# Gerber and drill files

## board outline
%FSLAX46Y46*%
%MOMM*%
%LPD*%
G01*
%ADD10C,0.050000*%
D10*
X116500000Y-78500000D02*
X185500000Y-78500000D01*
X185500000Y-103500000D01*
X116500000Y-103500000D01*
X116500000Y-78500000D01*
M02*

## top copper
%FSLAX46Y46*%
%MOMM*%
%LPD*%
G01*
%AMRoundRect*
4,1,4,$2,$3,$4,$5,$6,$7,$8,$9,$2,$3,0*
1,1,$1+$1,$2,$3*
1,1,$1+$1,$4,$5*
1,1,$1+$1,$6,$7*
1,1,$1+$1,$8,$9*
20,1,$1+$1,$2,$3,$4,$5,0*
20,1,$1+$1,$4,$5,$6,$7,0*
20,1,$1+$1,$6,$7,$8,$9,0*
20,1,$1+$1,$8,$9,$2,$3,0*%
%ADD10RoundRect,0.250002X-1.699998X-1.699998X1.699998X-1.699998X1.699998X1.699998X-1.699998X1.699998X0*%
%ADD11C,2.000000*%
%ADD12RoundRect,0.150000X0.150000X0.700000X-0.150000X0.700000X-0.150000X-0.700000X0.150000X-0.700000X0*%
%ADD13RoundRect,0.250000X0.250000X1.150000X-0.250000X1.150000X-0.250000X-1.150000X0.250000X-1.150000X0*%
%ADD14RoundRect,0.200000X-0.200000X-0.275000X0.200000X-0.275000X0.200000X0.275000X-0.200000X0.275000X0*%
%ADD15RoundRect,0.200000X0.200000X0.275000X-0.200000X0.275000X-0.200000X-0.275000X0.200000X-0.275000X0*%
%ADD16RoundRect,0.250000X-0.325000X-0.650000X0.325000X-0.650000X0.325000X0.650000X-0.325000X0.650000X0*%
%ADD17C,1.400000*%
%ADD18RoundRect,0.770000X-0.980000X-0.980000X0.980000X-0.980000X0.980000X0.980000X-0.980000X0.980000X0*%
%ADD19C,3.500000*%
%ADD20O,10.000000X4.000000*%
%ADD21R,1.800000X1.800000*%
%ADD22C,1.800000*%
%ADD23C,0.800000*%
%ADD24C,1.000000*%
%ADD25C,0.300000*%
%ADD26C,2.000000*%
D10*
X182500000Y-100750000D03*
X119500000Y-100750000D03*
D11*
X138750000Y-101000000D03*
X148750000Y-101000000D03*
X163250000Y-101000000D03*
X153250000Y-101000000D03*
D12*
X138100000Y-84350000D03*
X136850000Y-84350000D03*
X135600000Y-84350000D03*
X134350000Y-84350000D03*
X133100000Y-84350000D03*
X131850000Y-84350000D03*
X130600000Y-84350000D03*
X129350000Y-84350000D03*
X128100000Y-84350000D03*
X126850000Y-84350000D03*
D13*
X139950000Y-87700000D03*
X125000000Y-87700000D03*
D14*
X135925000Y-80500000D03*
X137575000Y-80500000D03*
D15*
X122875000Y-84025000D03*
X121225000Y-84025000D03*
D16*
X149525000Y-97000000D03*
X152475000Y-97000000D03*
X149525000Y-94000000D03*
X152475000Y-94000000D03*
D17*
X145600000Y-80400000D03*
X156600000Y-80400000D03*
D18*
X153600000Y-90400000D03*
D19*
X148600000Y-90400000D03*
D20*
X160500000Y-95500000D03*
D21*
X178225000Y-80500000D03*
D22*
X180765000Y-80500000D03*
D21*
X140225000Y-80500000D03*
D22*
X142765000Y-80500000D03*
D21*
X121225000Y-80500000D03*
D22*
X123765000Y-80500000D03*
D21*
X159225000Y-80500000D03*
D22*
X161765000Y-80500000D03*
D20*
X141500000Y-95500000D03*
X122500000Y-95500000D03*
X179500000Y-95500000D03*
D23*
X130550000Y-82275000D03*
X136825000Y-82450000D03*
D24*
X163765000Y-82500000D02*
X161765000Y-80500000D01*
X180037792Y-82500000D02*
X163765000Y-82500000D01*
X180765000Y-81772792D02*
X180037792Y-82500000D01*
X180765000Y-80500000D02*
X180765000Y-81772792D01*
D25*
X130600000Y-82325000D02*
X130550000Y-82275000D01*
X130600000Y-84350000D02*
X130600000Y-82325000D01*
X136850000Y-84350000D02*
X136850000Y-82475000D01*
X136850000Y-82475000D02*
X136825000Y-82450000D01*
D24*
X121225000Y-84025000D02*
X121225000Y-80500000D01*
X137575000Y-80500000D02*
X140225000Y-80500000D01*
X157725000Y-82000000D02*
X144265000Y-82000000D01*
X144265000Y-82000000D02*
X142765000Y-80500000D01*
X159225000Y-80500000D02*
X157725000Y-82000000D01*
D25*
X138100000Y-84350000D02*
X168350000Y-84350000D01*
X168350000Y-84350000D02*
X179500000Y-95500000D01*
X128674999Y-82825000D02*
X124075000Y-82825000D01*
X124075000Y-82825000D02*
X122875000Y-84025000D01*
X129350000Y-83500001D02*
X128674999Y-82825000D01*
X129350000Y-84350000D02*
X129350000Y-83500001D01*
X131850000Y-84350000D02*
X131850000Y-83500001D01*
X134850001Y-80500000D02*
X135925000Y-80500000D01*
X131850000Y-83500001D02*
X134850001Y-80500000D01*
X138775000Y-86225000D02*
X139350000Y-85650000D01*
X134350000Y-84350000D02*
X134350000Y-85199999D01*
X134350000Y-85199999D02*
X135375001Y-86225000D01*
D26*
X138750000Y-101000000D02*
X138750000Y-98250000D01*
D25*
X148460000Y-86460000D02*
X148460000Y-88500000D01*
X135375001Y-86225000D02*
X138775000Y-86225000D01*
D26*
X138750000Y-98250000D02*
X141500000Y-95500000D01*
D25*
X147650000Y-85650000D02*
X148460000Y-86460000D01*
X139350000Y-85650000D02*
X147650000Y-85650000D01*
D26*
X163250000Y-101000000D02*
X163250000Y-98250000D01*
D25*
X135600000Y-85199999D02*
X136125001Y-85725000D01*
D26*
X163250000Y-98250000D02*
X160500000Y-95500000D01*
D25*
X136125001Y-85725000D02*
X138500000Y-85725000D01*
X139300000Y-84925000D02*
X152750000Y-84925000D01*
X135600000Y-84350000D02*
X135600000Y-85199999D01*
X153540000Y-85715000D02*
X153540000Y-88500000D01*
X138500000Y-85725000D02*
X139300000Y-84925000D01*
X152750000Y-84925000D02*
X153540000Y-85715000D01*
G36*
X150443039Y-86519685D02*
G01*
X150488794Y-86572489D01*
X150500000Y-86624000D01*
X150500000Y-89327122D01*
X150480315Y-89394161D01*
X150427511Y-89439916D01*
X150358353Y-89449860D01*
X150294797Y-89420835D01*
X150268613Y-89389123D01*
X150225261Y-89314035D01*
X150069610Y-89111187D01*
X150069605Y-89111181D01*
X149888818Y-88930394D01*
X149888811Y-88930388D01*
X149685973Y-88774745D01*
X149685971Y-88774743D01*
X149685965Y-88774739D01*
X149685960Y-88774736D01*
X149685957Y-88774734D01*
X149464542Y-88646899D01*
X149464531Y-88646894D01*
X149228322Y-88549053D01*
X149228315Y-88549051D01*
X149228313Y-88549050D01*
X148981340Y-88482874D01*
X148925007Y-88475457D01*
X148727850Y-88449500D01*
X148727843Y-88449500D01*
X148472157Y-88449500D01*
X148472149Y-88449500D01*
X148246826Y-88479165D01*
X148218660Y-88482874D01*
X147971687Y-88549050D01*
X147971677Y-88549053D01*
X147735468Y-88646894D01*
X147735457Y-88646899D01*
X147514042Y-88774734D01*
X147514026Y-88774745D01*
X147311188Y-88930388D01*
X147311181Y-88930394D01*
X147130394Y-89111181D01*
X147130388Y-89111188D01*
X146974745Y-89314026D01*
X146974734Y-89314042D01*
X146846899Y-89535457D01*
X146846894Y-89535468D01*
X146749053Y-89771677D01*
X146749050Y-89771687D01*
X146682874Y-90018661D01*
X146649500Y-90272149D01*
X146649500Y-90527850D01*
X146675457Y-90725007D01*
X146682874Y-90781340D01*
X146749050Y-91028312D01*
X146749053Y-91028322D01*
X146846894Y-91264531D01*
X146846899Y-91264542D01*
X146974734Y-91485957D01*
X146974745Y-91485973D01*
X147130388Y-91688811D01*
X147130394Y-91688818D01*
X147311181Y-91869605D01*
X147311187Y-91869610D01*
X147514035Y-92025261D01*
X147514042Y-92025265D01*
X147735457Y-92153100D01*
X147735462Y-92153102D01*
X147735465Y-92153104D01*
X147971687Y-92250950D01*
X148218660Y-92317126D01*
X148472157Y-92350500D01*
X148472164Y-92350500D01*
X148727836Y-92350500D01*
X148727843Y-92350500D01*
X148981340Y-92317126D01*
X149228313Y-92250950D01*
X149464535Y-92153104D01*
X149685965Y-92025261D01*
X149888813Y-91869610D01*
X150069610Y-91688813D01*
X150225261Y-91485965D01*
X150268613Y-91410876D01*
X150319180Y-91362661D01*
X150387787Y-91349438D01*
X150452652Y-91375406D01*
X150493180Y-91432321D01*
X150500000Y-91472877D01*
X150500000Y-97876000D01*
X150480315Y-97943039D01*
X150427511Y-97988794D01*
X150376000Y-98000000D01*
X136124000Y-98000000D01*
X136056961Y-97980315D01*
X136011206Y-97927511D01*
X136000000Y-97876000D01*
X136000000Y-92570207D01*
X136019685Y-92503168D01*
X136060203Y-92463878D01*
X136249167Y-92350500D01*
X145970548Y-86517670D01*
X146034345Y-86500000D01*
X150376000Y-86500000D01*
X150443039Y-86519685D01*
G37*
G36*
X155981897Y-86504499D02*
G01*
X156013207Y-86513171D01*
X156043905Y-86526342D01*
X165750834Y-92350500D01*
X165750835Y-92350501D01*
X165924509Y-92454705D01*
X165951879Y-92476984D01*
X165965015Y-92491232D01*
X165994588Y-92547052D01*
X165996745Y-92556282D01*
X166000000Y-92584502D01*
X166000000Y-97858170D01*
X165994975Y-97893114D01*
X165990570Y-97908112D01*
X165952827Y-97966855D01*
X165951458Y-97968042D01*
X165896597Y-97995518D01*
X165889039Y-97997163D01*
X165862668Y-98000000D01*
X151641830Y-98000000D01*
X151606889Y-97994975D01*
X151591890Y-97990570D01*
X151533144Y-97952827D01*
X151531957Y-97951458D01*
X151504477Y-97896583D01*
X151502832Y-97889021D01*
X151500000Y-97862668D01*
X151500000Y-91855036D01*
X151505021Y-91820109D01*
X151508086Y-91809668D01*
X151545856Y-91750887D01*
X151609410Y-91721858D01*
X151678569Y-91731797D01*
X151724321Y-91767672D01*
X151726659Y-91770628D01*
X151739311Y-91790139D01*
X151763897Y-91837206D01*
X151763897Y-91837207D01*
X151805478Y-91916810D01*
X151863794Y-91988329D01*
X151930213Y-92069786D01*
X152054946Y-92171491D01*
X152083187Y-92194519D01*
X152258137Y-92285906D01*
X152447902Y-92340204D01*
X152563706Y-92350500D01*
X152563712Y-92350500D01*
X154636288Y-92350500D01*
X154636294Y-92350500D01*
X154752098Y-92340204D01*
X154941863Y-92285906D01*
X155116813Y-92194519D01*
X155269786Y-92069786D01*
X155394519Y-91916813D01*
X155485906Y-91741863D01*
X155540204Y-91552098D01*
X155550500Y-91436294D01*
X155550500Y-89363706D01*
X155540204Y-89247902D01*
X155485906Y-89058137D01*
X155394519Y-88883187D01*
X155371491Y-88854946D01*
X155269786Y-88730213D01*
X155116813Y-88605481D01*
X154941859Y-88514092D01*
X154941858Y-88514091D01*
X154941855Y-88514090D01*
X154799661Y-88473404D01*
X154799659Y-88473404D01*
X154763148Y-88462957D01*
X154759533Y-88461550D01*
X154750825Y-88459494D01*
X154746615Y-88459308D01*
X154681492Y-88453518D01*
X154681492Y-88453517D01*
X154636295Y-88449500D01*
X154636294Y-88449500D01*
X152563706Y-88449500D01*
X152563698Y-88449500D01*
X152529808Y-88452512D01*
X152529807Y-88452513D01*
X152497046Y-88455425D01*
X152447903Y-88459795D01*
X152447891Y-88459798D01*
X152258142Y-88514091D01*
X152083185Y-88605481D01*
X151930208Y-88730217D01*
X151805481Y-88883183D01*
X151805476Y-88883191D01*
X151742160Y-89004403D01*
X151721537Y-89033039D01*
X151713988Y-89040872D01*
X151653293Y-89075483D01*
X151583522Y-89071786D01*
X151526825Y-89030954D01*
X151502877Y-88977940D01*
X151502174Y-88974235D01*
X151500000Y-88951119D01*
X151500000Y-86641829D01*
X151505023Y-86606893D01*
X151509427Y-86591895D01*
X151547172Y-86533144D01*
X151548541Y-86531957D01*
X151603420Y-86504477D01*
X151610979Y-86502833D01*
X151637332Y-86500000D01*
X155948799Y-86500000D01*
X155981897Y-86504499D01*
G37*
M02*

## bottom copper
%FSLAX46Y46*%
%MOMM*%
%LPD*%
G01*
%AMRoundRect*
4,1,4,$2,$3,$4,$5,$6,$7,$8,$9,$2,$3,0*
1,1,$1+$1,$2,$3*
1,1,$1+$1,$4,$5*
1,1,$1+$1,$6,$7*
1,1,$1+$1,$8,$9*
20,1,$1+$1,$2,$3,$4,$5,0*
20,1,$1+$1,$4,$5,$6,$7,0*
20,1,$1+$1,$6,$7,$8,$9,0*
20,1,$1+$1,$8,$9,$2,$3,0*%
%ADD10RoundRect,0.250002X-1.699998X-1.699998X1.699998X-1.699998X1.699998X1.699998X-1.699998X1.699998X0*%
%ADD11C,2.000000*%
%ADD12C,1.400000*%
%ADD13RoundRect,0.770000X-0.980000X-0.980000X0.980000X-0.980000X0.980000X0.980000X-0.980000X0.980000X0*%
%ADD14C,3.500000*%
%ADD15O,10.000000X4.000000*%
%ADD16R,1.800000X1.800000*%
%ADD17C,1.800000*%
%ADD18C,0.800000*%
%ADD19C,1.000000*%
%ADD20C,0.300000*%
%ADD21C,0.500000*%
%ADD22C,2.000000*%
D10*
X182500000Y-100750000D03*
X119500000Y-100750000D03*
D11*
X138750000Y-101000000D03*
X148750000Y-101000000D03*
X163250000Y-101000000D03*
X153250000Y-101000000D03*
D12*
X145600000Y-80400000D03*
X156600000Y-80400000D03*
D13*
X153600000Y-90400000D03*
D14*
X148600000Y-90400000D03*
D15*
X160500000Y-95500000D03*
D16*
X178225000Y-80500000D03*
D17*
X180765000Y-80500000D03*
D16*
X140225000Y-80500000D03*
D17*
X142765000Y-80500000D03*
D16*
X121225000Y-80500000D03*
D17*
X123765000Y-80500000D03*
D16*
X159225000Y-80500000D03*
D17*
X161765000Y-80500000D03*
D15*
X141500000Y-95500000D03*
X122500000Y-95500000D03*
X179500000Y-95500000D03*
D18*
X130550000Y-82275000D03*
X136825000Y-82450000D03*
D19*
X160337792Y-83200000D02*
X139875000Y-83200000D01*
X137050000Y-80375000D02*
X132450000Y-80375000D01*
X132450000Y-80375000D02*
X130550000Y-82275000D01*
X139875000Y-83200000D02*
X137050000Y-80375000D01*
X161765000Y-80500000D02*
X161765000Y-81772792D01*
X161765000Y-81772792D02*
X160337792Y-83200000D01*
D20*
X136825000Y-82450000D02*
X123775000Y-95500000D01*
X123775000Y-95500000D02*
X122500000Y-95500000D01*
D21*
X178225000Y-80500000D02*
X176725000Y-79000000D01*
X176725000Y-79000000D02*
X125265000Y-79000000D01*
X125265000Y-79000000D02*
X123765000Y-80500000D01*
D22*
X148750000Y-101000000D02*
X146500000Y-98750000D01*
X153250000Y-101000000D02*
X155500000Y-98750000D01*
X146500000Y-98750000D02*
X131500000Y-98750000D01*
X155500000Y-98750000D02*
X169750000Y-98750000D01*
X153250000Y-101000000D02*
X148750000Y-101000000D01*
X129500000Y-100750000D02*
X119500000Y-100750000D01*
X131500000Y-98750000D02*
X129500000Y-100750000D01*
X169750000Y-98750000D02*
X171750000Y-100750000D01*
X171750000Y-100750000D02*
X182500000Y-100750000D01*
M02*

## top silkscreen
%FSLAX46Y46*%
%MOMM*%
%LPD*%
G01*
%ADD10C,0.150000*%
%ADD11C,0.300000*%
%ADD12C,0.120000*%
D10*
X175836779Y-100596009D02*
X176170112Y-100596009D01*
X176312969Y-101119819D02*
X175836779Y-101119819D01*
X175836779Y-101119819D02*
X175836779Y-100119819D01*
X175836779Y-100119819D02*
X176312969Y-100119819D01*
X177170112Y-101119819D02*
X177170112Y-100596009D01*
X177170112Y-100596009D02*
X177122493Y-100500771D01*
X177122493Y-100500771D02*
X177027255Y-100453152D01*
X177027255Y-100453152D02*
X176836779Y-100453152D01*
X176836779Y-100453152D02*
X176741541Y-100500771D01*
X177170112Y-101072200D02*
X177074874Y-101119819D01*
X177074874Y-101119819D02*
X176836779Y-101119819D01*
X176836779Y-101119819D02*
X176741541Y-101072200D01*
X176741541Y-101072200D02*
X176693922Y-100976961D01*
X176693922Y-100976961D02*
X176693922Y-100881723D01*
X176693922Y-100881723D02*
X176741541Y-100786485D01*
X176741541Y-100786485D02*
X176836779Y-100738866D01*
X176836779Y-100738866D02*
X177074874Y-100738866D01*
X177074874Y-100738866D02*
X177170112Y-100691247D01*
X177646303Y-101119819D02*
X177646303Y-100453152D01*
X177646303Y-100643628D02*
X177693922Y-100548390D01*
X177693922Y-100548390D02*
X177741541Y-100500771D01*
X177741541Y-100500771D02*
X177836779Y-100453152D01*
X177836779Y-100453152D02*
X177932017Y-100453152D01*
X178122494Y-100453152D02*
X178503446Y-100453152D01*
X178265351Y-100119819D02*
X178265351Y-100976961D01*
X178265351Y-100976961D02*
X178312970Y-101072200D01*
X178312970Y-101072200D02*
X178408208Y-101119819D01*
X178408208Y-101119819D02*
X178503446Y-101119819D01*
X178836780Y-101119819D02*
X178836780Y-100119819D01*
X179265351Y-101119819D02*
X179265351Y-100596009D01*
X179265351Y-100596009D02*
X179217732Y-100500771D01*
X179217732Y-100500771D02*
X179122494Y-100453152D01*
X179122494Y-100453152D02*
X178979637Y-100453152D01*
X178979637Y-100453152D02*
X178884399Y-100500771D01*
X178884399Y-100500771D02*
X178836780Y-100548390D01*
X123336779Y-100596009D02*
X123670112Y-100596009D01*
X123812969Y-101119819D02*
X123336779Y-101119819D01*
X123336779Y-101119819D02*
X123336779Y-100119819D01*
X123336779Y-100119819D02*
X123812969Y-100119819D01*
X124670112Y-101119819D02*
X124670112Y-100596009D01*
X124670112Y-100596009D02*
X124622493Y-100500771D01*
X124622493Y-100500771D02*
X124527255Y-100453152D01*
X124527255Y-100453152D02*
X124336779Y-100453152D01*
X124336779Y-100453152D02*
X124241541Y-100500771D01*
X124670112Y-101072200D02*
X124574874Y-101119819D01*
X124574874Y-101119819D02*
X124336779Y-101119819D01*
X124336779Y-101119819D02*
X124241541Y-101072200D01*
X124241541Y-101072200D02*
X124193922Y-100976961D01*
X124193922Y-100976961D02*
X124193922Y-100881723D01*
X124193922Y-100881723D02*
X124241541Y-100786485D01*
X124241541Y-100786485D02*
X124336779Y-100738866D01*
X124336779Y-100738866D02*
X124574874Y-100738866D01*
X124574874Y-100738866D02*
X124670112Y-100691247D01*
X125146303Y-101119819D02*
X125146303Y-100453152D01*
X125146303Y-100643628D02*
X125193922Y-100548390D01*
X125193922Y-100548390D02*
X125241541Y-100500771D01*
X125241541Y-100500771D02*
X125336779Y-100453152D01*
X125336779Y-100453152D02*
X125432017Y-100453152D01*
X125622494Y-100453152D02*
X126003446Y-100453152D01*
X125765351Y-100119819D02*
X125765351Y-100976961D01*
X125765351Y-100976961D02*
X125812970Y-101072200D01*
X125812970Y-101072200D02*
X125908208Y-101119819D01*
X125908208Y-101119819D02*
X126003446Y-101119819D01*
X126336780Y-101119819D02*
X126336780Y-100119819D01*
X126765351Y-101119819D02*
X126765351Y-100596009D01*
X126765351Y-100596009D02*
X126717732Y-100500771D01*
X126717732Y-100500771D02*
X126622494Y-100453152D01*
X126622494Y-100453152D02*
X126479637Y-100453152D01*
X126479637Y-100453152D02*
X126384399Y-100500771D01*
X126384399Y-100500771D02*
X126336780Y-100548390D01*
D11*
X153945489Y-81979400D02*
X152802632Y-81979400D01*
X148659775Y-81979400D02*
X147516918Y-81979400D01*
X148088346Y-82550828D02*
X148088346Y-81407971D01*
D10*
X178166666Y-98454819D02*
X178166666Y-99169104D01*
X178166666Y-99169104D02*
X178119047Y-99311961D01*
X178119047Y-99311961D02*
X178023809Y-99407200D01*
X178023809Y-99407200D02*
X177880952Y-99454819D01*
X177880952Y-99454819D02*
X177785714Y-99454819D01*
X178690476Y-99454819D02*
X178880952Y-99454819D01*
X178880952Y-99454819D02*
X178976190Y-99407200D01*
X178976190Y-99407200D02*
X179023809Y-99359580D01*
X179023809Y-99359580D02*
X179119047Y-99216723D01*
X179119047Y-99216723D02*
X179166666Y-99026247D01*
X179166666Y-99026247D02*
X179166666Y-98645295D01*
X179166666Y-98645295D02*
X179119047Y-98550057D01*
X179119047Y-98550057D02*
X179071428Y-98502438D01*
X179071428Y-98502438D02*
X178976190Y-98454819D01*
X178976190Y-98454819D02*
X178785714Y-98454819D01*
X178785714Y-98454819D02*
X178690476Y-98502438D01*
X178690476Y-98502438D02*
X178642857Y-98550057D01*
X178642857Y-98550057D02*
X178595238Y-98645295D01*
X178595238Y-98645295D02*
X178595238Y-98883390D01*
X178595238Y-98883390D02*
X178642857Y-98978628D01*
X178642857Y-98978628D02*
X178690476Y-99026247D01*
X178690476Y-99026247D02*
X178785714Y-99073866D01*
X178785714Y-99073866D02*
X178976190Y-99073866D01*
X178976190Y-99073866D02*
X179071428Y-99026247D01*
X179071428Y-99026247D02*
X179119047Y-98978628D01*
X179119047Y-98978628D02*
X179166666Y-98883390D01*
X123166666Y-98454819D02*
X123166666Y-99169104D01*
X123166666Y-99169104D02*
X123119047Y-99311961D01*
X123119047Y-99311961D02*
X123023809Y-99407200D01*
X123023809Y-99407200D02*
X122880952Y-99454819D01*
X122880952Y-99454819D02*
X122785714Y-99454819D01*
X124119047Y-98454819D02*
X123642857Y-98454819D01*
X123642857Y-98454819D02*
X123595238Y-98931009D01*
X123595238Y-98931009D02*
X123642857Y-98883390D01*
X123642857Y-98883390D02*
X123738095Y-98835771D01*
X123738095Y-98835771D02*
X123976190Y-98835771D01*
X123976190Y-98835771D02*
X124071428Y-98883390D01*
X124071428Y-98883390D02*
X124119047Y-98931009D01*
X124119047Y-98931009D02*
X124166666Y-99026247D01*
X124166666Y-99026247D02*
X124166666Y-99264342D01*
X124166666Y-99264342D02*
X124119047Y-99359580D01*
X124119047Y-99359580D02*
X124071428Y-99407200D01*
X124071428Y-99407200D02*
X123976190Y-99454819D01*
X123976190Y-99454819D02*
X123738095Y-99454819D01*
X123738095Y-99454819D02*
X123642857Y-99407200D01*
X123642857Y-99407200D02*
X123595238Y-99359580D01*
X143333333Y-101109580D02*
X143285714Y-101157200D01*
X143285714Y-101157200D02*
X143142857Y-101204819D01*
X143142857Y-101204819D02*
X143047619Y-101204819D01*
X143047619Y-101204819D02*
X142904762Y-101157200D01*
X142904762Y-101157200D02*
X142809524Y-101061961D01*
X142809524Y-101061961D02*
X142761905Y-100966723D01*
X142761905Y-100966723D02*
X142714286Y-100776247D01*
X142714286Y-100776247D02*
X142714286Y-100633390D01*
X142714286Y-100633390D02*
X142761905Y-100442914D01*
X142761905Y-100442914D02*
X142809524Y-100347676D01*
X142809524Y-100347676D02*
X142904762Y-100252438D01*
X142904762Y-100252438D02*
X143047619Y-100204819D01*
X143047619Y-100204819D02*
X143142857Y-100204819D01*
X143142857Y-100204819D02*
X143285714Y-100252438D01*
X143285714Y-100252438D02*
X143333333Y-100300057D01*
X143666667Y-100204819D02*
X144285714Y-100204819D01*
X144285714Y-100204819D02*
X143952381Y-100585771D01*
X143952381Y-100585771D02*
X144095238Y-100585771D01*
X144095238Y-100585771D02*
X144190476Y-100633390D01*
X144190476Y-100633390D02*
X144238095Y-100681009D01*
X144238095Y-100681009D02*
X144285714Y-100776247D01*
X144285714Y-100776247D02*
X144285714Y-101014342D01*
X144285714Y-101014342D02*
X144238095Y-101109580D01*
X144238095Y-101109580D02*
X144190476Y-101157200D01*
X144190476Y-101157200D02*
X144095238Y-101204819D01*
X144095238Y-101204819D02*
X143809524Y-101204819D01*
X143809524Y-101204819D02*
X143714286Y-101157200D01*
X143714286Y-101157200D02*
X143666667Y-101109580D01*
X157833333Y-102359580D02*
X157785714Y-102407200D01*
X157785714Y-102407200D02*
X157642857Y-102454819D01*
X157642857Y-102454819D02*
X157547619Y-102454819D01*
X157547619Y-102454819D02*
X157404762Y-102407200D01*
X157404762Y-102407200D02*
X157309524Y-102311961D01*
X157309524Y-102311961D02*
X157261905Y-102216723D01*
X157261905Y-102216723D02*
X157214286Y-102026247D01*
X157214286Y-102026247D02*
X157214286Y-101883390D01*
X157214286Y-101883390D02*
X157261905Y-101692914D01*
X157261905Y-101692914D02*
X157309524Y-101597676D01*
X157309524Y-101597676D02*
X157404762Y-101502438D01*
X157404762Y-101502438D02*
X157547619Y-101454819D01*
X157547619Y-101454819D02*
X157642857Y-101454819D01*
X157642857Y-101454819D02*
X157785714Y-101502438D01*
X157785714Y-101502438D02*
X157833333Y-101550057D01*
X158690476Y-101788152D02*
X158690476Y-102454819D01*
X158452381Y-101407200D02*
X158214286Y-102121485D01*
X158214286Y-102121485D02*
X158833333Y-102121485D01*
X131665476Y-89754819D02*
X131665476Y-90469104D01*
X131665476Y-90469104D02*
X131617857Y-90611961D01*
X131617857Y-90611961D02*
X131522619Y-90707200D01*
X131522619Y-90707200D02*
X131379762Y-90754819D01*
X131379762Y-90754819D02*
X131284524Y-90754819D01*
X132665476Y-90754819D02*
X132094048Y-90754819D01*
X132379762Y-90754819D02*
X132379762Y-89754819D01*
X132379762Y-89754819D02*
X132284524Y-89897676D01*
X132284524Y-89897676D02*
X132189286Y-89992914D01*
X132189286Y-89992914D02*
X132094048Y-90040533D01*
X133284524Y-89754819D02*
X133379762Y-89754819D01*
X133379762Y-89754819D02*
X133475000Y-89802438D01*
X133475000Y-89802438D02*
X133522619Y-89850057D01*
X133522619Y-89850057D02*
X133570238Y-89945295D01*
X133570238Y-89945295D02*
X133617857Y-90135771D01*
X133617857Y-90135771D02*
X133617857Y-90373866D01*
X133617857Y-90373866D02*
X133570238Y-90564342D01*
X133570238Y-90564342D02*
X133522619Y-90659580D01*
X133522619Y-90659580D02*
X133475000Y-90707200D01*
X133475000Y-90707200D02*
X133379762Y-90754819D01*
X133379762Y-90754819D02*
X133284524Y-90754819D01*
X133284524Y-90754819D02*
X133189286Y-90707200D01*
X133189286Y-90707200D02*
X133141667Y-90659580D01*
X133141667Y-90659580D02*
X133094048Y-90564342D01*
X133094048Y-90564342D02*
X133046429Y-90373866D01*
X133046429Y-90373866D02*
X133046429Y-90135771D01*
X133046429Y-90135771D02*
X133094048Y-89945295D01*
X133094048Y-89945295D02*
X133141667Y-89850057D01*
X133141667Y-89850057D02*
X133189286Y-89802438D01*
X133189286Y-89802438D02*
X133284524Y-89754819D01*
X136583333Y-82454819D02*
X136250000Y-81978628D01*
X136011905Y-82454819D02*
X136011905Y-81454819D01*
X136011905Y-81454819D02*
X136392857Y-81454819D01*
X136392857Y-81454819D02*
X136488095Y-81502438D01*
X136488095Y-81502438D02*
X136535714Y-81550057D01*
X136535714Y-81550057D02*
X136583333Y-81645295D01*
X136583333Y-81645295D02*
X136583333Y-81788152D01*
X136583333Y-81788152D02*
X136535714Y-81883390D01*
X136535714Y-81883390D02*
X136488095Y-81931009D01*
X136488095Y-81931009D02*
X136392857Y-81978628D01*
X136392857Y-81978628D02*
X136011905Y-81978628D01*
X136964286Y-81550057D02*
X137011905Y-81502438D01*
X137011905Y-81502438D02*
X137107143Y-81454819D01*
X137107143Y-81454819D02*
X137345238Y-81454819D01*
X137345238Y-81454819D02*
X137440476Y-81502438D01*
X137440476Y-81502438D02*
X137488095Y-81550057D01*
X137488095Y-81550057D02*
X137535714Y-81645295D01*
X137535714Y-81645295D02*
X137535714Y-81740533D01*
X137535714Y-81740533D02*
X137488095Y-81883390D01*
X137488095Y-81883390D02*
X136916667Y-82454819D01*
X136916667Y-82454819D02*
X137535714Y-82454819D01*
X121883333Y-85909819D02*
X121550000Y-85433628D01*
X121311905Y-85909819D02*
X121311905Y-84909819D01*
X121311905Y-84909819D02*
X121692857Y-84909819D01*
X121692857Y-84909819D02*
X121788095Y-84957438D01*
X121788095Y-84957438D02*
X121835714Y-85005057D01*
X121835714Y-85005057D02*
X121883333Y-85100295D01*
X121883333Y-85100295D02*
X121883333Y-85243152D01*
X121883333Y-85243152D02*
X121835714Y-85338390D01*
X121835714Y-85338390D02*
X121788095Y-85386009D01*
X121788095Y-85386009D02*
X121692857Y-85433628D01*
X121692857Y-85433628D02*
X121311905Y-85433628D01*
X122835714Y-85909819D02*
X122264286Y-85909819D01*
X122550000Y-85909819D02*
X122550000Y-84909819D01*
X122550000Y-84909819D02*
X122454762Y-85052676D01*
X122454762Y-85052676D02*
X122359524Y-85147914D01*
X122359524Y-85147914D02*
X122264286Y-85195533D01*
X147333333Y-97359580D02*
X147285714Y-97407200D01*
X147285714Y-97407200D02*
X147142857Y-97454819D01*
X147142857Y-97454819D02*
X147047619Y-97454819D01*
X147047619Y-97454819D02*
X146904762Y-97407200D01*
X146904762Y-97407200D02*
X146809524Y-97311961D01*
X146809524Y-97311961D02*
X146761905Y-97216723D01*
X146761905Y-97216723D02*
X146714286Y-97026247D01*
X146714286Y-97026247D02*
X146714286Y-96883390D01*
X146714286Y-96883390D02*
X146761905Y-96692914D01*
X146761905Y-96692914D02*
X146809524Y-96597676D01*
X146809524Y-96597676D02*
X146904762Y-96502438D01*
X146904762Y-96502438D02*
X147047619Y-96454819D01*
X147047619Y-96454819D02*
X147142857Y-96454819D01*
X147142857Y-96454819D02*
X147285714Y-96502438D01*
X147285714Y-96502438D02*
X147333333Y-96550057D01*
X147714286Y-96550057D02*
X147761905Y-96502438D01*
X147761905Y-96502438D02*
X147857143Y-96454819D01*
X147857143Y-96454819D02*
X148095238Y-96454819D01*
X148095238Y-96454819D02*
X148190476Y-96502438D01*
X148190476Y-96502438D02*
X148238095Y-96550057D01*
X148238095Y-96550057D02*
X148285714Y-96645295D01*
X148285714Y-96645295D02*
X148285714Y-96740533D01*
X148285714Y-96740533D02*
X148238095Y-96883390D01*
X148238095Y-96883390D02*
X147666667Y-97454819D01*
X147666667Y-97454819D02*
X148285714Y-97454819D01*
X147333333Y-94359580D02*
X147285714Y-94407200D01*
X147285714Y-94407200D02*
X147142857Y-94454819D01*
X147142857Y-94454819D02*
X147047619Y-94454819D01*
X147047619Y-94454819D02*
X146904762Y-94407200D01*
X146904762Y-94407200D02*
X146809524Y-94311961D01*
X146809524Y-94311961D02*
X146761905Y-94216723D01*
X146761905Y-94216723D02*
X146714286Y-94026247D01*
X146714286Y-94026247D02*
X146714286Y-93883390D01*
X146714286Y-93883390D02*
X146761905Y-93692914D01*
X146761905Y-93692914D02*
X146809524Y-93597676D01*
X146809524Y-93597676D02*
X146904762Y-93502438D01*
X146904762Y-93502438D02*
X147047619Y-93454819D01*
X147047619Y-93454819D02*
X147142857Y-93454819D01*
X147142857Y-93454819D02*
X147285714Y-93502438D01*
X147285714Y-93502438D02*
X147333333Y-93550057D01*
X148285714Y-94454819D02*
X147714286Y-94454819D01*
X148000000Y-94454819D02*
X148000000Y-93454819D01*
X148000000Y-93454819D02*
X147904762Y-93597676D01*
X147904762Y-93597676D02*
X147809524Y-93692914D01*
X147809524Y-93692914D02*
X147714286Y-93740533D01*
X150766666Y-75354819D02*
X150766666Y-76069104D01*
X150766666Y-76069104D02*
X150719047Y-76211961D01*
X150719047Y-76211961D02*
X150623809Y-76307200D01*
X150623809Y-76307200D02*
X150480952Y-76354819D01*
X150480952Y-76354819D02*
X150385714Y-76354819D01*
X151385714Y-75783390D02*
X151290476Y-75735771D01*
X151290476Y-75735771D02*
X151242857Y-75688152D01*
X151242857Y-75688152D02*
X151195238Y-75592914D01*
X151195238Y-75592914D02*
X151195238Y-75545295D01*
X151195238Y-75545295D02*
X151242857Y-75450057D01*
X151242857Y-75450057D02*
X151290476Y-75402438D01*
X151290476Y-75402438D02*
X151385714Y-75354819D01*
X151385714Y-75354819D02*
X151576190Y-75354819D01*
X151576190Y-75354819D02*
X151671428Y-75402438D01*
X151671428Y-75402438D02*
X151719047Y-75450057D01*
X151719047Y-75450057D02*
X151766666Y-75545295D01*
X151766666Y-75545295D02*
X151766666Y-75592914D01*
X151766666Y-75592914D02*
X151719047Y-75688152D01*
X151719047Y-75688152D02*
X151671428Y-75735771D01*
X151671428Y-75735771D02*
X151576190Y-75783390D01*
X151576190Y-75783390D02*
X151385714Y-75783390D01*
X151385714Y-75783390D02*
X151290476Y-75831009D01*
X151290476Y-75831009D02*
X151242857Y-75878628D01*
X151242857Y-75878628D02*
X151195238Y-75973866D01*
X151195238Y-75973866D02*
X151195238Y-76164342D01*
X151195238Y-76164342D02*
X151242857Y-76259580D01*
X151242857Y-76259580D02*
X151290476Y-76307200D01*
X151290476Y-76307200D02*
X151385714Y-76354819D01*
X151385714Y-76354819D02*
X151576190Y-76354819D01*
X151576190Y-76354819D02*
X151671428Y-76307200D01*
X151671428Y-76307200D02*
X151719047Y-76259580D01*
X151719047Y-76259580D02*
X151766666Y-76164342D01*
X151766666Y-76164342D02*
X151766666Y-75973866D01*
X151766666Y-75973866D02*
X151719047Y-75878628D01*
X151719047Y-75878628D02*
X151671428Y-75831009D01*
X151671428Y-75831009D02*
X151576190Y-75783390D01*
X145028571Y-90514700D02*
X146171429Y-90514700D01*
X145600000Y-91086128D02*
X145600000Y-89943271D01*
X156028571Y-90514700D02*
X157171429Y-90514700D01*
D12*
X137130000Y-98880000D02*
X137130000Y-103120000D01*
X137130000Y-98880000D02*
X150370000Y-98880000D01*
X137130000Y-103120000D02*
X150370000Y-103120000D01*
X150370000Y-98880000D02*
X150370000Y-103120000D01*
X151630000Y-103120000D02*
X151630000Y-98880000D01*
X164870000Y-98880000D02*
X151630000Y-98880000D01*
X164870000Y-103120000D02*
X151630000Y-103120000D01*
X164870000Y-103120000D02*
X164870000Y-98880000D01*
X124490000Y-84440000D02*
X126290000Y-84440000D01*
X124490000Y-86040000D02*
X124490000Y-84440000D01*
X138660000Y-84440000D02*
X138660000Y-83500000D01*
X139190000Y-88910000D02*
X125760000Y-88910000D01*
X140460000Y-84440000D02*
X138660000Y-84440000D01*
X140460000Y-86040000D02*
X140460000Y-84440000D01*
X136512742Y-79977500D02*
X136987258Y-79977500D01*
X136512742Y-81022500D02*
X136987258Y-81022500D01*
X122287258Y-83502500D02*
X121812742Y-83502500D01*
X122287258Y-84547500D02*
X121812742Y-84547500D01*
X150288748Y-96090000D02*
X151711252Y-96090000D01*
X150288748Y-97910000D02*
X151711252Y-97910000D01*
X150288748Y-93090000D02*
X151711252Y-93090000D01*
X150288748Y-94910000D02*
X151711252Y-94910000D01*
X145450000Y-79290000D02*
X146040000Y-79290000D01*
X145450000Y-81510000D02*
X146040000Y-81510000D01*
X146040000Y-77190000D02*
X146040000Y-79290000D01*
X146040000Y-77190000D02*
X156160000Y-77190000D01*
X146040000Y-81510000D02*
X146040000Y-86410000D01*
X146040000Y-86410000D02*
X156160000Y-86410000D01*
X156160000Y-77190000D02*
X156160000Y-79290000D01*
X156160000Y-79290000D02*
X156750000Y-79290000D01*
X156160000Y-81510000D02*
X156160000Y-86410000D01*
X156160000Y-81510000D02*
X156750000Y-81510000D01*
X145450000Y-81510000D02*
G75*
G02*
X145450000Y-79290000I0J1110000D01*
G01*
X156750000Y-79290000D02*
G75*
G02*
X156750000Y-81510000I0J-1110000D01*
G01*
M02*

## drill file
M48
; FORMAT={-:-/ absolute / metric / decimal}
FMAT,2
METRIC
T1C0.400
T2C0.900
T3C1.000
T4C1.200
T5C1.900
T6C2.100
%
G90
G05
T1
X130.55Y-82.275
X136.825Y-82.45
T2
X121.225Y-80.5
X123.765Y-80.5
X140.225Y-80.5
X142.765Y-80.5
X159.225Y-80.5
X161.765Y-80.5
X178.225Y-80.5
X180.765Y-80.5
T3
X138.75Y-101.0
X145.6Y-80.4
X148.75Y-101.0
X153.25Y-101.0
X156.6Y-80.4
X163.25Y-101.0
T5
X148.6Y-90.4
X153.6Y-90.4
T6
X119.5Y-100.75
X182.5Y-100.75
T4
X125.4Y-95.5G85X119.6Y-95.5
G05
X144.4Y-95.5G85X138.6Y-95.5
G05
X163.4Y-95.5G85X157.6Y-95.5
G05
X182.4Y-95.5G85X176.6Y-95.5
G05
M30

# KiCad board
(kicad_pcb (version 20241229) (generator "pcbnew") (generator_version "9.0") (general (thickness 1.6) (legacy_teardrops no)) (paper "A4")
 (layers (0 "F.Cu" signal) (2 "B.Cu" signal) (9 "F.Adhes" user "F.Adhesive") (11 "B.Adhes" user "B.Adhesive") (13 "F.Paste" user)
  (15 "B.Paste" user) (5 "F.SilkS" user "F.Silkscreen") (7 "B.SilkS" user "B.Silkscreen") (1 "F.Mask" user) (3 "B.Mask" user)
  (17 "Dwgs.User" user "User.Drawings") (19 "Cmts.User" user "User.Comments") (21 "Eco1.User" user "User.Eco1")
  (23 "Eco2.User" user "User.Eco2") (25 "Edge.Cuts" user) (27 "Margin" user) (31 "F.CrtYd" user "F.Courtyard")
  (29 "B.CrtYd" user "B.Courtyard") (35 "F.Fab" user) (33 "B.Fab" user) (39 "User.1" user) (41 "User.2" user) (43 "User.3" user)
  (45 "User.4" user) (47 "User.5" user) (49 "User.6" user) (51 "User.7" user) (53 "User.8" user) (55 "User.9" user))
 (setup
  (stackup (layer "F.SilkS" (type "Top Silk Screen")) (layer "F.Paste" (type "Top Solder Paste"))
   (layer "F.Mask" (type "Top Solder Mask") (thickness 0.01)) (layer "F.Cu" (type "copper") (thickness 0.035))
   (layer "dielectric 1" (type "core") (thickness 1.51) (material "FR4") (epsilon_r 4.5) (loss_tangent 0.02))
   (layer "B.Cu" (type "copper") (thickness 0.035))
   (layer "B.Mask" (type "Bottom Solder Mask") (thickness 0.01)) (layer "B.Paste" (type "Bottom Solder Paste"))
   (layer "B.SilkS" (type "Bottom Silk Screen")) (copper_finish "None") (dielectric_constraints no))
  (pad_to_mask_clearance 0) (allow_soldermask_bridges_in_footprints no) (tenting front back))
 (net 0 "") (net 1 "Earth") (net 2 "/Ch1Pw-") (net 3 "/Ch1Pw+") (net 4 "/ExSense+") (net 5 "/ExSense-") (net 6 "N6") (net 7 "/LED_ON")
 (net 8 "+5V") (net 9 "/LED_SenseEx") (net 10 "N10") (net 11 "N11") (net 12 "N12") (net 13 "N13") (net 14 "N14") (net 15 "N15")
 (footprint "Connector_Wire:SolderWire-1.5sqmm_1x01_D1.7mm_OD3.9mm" (layer "F.Cu") (at 182.5 100.75)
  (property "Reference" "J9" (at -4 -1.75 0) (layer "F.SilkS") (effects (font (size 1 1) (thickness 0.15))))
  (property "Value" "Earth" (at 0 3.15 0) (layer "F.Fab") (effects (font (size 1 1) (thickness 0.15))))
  (pad "1" thru_hole roundrect (at 0 0) (size 3.9 3.9) (drill 2.1) (layers "*.Cu" "*.Mask") (remove_unused_layers no)
   (roundrect_rratio 0.064103) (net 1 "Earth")))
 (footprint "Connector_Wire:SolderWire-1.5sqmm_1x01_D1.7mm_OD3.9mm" (layer "F.Cu") (at 119.5 100.75)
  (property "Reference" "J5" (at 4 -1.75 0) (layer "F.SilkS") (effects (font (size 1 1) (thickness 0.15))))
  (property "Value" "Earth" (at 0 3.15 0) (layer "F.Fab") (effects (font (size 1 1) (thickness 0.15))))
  (pad "1" thru_hole roundrect (at 0 0) (size 3.9 3.9) (drill 2.1) (layers "*.Cu" "*.Mask") (remove_unused_layers no)
   (roundrect_rratio 0.064103) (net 1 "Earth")))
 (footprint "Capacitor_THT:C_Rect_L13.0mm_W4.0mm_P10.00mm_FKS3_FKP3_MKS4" (layer "F.Cu") (at 138.75 101)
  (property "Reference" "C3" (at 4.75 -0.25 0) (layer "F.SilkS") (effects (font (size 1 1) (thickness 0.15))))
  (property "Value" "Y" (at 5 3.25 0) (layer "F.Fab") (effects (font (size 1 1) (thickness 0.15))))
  (fp_line (start -1.62 -2.12) (end -1.62 2.12) (stroke (width 0.12) (type solid)) (layer "F.SilkS"))
  (fp_line (start -1.62 -2.12) (end 11.62 -2.12) (stroke (width 0.12) (type solid)) (layer "F.SilkS"))
  (fp_line (start -1.62 2.12) (end 11.62 2.12) (stroke (width 0.12) (type solid)) (layer "F.SilkS"))
  (fp_line (start 11.62 -2.12) (end 11.62 2.12) (stroke (width 0.12) (type solid)) (layer "F.SilkS"))
  (pad "1" thru_hole circle (at 0 0) (size 2 2) (drill 1) (layers "*.Cu" "*.Mask") (remove_unused_layers no) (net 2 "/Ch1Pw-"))
  (pad "2" thru_hole circle (at 10 0) (size 2 2) (drill 1) (layers "*.Cu" "*.Mask") (remove_unused_layers no) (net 1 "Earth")))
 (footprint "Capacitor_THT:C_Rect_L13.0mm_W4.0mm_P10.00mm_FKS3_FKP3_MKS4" (layer "F.Cu") (at 163.25 101 180)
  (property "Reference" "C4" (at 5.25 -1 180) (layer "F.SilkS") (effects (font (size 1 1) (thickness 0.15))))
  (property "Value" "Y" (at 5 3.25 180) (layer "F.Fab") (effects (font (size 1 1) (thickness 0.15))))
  (fp_line (start 11.62 -2.12) (end 11.62 2.12) (stroke (width 0.12) (type solid)) (layer "F.SilkS"))
  (fp_line (start -1.62 2.12) (end 11.62 2.12) (stroke (width 0.12) (type solid)) (layer "F.SilkS"))
  (fp_line (start -1.62 -2.12) (end 11.62 -2.12) (stroke (width 0.12) (type solid)) (layer "F.SilkS"))
  (fp_line (start -1.62 -2.12) (end -1.62 2.12) (stroke (width 0.12) (type solid)) (layer "F.SilkS"))
  (pad "1" thru_hole circle (at 0 0 180) (size 2 2) (drill 1) (layers "*.Cu" "*.Mask") (remove_unused_layers no) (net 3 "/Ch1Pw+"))
  (pad "2" thru_hole circle (at 10 0 180) (size 2 2) (drill 1) (layers "*.Cu" "*.Mask") (remove_unused_layers no) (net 1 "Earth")))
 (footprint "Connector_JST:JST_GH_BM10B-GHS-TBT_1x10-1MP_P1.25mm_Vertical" (layer "F.Cu") (at 132.475 86.3 180)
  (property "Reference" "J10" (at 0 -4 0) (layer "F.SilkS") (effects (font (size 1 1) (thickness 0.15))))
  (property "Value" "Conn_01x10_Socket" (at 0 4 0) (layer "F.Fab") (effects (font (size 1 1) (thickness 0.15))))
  (fp_line (start 7.985 1.86) (end 6.185 1.86) (stroke (width 0.12) (type solid)) (layer "F.SilkS"))
  (fp_line (start 7.985 0.26) (end 7.985 1.86) (stroke (width 0.12) (type solid)) (layer "F.SilkS"))
  (fp_line (start -6.185 1.86) (end -6.185 2.8) (stroke (width 0.12) (type solid)) (layer "F.SilkS"))
  (fp_line (start -6.715 -2.61) (end 6.715 -2.61) (stroke (width 0.12) (type solid)) (layer "F.SilkS"))
  (fp_line (start -7.985 1.86) (end -6.185 1.86) (stroke (width 0.12) (type solid)) (layer "F.SilkS"))
  (fp_line (start -7.985 0.26) (end -7.985 1.86) (stroke (width 0.12) (type solid)) (layer "F.SilkS"))
  (pad "1" smd roundrect (at -5.625 1.95 180) (size 0.6 1.7) (layers "F.Cu" "F.Mask" "F.Paste") (roundrect_rratio 0.25) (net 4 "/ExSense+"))
  (pad "2" smd roundrect (at -4.375 1.95 180) (size 0.6 1.7) (layers "F.Cu" "F.Mask" "F.Paste") (roundrect_rratio 0.25) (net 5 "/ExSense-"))
  (pad "3" smd roundrect (at -3.125 1.95 180) (size 0.6 1.7) (layers "F.Cu" "F.Mask" "F.Paste") (roundrect_rratio 0.25) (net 3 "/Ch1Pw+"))
  (pad "4" smd roundrect (at -1.875 1.95 180) (size 0.6 1.7) (layers "F.Cu" "F.Mask" "F.Paste") (roundrect_rratio 0.25) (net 2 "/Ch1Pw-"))
  (pad "5" smd roundrect (at -0.625 1.95 180) (size 0.6 1.7) (layers "F.Cu" "F.Mask" "F.Paste") (roundrect_rratio 0.25) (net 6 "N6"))
  (pad "6" smd roundrect (at 0.625 1.95 180) (size 0.6 1.7) (layers "F.Cu" "F.Mask" "F.Paste") (roundrect_rratio 0.25) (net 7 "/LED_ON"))
  (pad "7" smd roundrect (at 1.875 1.95 180) (size 0.6 1.7) (layers "F.Cu" "F.Mask" "F.Paste") (roundrect_rratio 0.25) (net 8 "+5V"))
  (pad "8" smd roundrect (at 3.125 1.95 180) (size 0.6 1.7) (layers "F.Cu" "F.Mask" "F.Paste") (roundrect_rratio 0.25)
   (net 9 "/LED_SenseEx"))
  (pad "9" smd roundrect (at 4.375 1.95 180) (size 0.6 1.7) (layers "F.Cu" "F.Mask" "F.Paste") (roundrect_rratio 0.25) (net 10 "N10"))
  (pad "10" smd roundrect (at 5.625 1.95 180) (size 0.6 1.7) (layers "F.Cu" "F.Mask" "F.Paste") (roundrect_rratio 0.25) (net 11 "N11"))
  (pad "MP" smd roundrect (at -7.475 -1.4 180) (size 1 2.8) (layers "F.Cu" "F.Mask" "F.Paste") (roundrect_rratio 0.25))
  (pad "MP" smd roundrect (at 7.475 -1.4 180) (size 1 2.8) (layers "F.Cu" "F.Mask" "F.Paste") (roundrect_rratio 0.25)))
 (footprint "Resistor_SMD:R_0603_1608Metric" (layer "F.Cu") (at 136.75 80.5)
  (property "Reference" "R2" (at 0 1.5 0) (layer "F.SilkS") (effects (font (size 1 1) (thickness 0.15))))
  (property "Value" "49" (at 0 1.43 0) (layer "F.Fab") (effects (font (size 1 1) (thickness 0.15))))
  (fp_line (start -0.237258 -0.5225) (end 0.237258 -0.5225) (stroke (width 0.12) (type solid)) (layer "F.SilkS"))
  (fp_line (start -0.237258 0.5225) (end 0.237258 0.5225) (stroke (width 0.12) (type solid)) (layer "F.SilkS"))
  (pad "1" smd roundrect (at -0.825 0) (size 0.8 0.95) (layers "F.Cu" "F.Mask" "F.Paste") (roundrect_rratio 0.25) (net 7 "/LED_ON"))
  (pad "2" smd roundrect (at 0.825 0) (size 0.8 0.95) (layers "F.Cu" "F.Mask" "F.Paste") (roundrect_rratio 0.25) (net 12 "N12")))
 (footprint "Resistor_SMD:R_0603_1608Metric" (layer "F.Cu") (at 122.05 84.025 180)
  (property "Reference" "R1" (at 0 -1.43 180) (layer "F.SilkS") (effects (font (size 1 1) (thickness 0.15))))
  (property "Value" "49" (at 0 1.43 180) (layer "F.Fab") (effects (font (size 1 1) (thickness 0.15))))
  (fp_line (start -0.237258 0.5225) (end 0.237258 0.5225) (stroke (width 0.12) (type solid)) (layer "F.SilkS"))
  (fp_line (start -0.237258 -0.5225) (end 0.237258 -0.5225) (stroke (width 0.12) (type solid)) (layer "F.SilkS"))
  (pad "1" smd roundrect (at -0.825 0 180) (size 0.8 0.95) (layers "F.Cu" "F.Mask" "F.Paste") (roundrect_rratio 0.25) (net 9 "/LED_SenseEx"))
  (pad "2" smd roundrect (at 0.825 0 180) (size 0.8 0.95) (layers "F.Cu" "F.Mask" "F.Paste") (roundrect_rratio 0.25) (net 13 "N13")))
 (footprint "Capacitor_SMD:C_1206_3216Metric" (layer "F.Cu") (at 151 97)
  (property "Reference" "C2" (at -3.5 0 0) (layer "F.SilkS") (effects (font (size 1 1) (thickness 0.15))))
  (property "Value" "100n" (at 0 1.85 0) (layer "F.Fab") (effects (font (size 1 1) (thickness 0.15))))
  (fp_line (start -0.711252 -0.91) (end 0.711252 -0.91) (stroke (width 0.12) (type solid)) (layer "F.SilkS"))
  (fp_line (start -0.711252 0.91) (end 0.711252 0.91) (stroke (width 0.12) (type solid)) (layer "F.SilkS"))
  (pad "1" smd roundrect (at -1.475 0) (size 1.15 1.8) (layers "F.Cu" "F.Mask" "F.Paste") (roundrect_rratio 0.217391) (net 2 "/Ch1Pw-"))
  (pad "2" smd roundrect (at 1.475 0) (size 1.15 1.8) (layers "F.Cu" "F.Mask" "F.Paste") (roundrect_rratio 0.217391) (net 3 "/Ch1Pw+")))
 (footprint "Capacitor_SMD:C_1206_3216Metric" (layer "F.Cu") (at 151 94)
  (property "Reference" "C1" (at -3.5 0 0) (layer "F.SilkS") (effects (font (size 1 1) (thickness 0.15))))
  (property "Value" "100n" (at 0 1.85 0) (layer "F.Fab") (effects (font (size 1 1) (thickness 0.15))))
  (fp_line (start -0.711252 -0.91) (end 0.711252 -0.91) (stroke (width 0.12) (type solid)) (layer "F.SilkS"))
  (fp_line (start -0.711252 0.91) (end 0.711252 0.91) (stroke (width 0.12) (type solid)) (layer "F.SilkS"))
  (pad "1" smd roundrect (at -1.475 0) (size 1.15 1.8) (layers "F.Cu" "F.Mask" "F.Paste") (roundrect_rratio 0.217391) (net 2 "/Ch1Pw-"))
  (pad "2" smd roundrect (at 1.475 0) (size 1.15 1.8) (layers "F.Cu" "F.Mask" "F.Paste") (roundrect_rratio 0.217391) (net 3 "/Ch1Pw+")))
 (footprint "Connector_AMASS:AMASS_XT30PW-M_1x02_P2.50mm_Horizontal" (layer "F.Cu") (at 153.6 90.4)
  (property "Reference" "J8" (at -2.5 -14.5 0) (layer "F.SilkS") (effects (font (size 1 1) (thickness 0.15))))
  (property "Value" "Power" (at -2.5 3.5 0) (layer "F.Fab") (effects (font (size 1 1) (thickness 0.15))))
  (fp_line (start -8.15 -11.11) (end -7.56 -11.11) (stroke (width 0.12) (type solid)) (layer "F.SilkS"))
  (fp_line (start -8.15 -8.89) (end -7.56 -8.89) (stroke (width 0.12) (type solid)) (layer "F.SilkS"))
  (fp_line (start -7.56 -13.21) (end -7.56 -11.11) (stroke (width 0.12) (type solid)) (layer "F.SilkS"))
  (fp_line (start -7.56 -13.21) (end 2.56 -13.21) (stroke (width 0.12) (type solid)) (layer "F.SilkS"))
  (fp_line (start -7.56 -8.89) (end -7.56 -3.99) (stroke (width 0.12) (type solid)) (layer "F.SilkS"))
  (fp_line (start -7.56 -3.99) (end 2.56 -3.99) (stroke (width 0.12) (type solid)) (layer "F.SilkS"))
  (fp_line (start 2.56 -13.21) (end 2.56 -11.11) (stroke (width 0.12) (type solid)) (layer "F.SilkS"))
  (fp_line (start 2.56 -11.11) (end 3.15 -11.11) (stroke (width 0.12) (type solid)) (layer "F.SilkS"))
  (fp_line (start 2.56 -8.89) (end 2.56 -3.99) (stroke (width 0.12) (type solid)) (layer "F.SilkS"))
  (fp_line (start 2.56 -8.89) (end 3.15 -8.89) (stroke (width 0.12) (type solid)) (layer "F.SilkS"))
  (fp_arc (start -8.15 -8.89) (mid -9.26 -10) (end -8.15 -11.11) (stroke (width 0.12) (type solid)) (layer "F.SilkS"))
  (fp_arc (start 3.15 -11.11) (mid 4.26 -10) (end 3.15 -8.89) (stroke (width 0.12) (type solid)) (layer "F.SilkS"))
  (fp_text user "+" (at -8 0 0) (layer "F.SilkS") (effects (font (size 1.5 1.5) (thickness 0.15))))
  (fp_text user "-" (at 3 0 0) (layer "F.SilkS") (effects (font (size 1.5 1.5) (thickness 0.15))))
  (pad "" thru_hole circle (at -8 -10) (size 1.4 1.4) (drill 1) (layers "*.Cu" "*.Mask") (remove_unused_layers no))
  (pad "" thru_hole circle (at 3 -10) (size 1.4 1.4) (drill 1) (layers "*.Cu" "*.Mask") (remove_unused_layers no))
  (pad "1" thru_hole roundrect (at 0 0) (size 3.5 3.5) (drill 1.9) (layers "*.Cu" "*.Mask") (remove_unused_layers no)
   (roundrect_rratio 0.22) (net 2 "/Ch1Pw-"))
  (pad "2" thru_hole circle (at -5 0) (size 3.5 3.5) (drill 1.9) (layers "*.Cu" "*.Mask") (remove_unused_layers no) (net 3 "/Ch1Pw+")))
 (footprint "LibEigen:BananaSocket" (layer "B.Cu") (at 160.5 95.5 180)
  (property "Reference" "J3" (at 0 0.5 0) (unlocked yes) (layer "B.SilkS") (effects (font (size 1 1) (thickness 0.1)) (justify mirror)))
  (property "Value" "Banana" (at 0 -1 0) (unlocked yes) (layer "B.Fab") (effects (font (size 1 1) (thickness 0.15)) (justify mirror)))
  (pad "1" thru_hole oval (at 0 0 180) (size 10 4) (drill oval 7 1.2) (layers "*.Cu" "*.Mask") (remove_unused_layers no) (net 3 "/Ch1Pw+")))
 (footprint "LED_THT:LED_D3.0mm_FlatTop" (layer "B.Cu") (at 178.225 80.5)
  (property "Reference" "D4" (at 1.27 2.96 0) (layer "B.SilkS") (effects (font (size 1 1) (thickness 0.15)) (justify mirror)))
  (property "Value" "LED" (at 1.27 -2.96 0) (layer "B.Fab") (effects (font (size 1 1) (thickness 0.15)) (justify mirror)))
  (pad "1" thru_hole rect (at 0 0) (size 1.8 1.8) (drill 0.9) (layers "*.Cu" "*.Mask") (remove_unused_layers no) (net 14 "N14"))
  (pad "2" thru_hole circle (at 2.54 0) (size 1.8 1.8) (drill 0.9) (layers "*.Cu" "*.Mask") (remove_unused_layers no) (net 8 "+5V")))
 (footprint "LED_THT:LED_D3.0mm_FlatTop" (layer "B.Cu") (at 140.225 80.5)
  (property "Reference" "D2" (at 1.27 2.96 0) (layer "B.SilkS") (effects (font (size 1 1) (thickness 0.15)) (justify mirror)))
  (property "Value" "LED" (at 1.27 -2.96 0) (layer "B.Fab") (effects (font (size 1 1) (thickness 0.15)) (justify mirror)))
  (pad "1" thru_hole rect (at 0 0) (size 1.8 1.8) (drill 0.9) (layers "*.Cu" "*.Mask") (remove_unused_layers no) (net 12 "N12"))
  (pad "2" thru_hole circle (at 2.54 0) (size 1.8 1.8) (drill 0.9) (layers "*.Cu" "*.Mask") (remove_unused_layers no) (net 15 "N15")))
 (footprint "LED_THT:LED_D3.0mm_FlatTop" (layer "B.Cu") (at 121.225 80.5)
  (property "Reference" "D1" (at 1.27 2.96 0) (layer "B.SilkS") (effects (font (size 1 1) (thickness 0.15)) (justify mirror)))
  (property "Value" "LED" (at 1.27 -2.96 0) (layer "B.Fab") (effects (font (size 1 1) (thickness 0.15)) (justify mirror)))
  (pad "1" thru_hole rect (at 0 0) (size 1.8 1.8) (drill 0.9) (layers "*.Cu" "*.Mask") (remove_unused_layers no) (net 13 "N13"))
  (pad "2" thru_hole circle (at 2.54 0) (size 1.8 1.8) (drill 0.9) (layers "*.Cu" "*.Mask") (remove_unused_layers no) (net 14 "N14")))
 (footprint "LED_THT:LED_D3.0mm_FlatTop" (layer "B.Cu") (at 159.225 80.5)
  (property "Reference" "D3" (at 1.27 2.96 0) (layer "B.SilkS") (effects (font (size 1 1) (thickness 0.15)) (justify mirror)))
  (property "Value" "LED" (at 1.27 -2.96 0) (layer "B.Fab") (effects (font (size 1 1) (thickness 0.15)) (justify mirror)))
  (pad "1" thru_hole rect (at 0 0) (size 1.8 1.8) (drill 0.9) (layers "*.Cu" "*.Mask") (remove_unused_layers no) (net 15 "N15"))
  (pad "2" thru_hole circle (at 2.54 0) (size 1.8 1.8) (drill 0.9) (layers "*.Cu" "*.Mask") (remove_unused_layers no) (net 8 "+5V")))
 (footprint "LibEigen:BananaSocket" (layer "B.Cu") (at 141.5 95.5 180)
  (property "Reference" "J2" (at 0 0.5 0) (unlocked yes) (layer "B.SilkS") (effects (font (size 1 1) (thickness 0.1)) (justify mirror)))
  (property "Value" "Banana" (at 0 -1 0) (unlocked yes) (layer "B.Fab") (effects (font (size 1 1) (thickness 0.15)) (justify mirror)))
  (pad "1" thru_hole oval (at 0 0 180) (size 10 4) (drill oval 7 1.2) (layers "*.Cu" "*.Mask") (remove_unused_layers no) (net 2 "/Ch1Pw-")))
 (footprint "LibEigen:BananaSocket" (layer "B.Cu") (at 122.5 95.5 180)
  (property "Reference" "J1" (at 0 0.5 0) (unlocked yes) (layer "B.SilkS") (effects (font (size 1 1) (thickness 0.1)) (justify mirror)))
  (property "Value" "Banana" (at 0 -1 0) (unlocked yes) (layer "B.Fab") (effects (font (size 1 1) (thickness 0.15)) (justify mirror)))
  (pad "1" thru_hole oval (at 0 0 180) (size 10 4) (drill oval 7 1.2) (layers "*.Cu" "*.Mask") (remove_unused_layers no) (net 5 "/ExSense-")))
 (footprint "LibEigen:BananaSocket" (layer "B.Cu") (at 179.5 95.5 180)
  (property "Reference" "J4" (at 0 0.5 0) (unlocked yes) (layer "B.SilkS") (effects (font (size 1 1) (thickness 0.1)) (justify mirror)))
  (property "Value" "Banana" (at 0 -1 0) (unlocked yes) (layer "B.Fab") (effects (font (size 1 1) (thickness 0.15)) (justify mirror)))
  (pad "1" thru_hole oval (at 0 0 180) (size 10 4) (drill oval 7 1.2) (layers "*.Cu" "*.Mask") (remove_unused_layers no) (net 4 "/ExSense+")))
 (gr_rect (start 116.5 78.5) (end 185.5 103.5) (stroke (width 0.05) (type default)) (fill no) (layer "Edge.Cuts"))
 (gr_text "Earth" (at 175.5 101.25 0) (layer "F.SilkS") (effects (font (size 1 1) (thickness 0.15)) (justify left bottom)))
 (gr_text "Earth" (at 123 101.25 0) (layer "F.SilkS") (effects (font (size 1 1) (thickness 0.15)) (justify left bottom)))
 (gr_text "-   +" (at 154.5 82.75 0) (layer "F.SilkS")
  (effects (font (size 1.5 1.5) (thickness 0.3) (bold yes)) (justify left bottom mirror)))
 (segment (start 163.765 82.5) (end 161.765 80.5) (width 1) (layer "F.Cu") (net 8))
 (segment (start 180.037792 82.5) (end 163.765 82.5) (width 1) (layer "F.Cu") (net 8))
 (segment (start 180.765 81.772792) (end 180.037792 82.5) (width 1) (layer "F.Cu") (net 8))
 (segment (start 180.765 80.5) (end 180.765 81.772792) (width 1) (layer "F.Cu") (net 8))
 (segment (start 130.6 82.325) (end 130.55 82.275) (width 0.3) (layer "F.Cu") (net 8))
 (segment (start 130.6 84.35) (end 130.6 82.325) (width 0.3) (layer "F.Cu") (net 8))
 (via (at 130.55 82.275) (size 0.8) (drill 0.4) (layers "F.Cu" "B.Cu") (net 8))
 (segment (start 160.337792 83.2) (end 139.875 83.2) (width 1) (layer "B.Cu") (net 8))
 (segment (start 137.05 80.375) (end 132.45 80.375) (width 1) (layer "B.Cu") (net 8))
 (segment (start 132.45 80.375) (end 130.55 82.275) (width 1) (layer "B.Cu") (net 8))
 (segment (start 139.875 83.2) (end 137.05 80.375) (width 1) (layer "B.Cu") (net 8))
 (segment (start 161.765 80.5) (end 161.765 81.772792) (width 1) (layer "B.Cu") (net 8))
 (segment (start 161.765 81.772792) (end 160.337792 83.2) (width 1) (layer "B.Cu") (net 8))
 (segment (start 136.85 84.35) (end 136.85 82.475) (width 0.3) (layer "F.Cu") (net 5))
 (segment (start 136.85 82.475) (end 136.825 82.45) (width 0.3) (layer "F.Cu") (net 5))
 (via (at 136.825 82.45) (size 0.8) (drill 0.4) (layers "F.Cu" "B.Cu") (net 5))
 (segment (start 136.825 82.45) (end 123.775 95.5) (width 0.3) (layer "B.Cu") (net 5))
 (segment (start 123.775 95.5) (end 122.5 95.5) (width 0.3) (layer "B.Cu") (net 5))
 (segment (start 178.225 80.5) (end 176.725 79) (width 0.5) (layer "B.Cu") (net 14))
 (segment (start 176.725 79) (end 125.265 79) (width 0.5) (layer "B.Cu") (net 14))
 (segment (start 125.265 79) (end 123.765 80.5) (width 0.5) (layer "B.Cu") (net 14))
 (segment (start 121.225 84.025) (end 121.225 80.5) (width 1) (layer "F.Cu") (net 13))
 (segment (start 137.575 80.5) (end 140.225 80.5) (width 1) (layer "F.Cu") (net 12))
 (segment (start 157.725 82) (end 144.265 82) (width 1) (layer "F.Cu") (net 15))
 (segment (start 144.265 82) (end 142.765 80.5) (width 1) (layer "F.Cu") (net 15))
 (segment (start 159.225 80.5) (end 157.725 82) (width 1) (layer "F.Cu") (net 15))
 (segment (start 138.1 84.35) (end 168.35 84.35) (width 0.3) (layer "F.Cu") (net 4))
 (segment (start 168.35 84.35) (end 179.5 95.5) (width 0.3) (layer "F.Cu") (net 4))
 (segment (start 128.674999 82.825) (end 124.075 82.825) (width 0.3) (layer "F.Cu") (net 9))
 (segment (start 124.075 82.825) (end 122.875 84.025) (width 0.3) (layer "F.Cu") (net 9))
 (segment (start 129.35 83.500001) (end 128.674999 82.825) (width 0.3) (layer "F.Cu") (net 9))
 (segment (start 129.35 84.35) (end 129.35 83.500001) (width 0.3) (layer "F.Cu") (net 9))
 (segment (start 131.85 84.35) (end 131.85 83.500001) (width 0.3) (layer "F.Cu") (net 7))
 (segment (start 134.850001 80.5) (end 135.925 80.5) (width 0.3) (layer "F.Cu") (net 7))
 (segment (start 131.85 83.500001) (end 134.850001 80.5) (width 0.3) (layer "F.Cu") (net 7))
 (segment (start 138.775 86.225) (end 139.35 85.65) (width 0.3) (layer "F.Cu") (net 2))
 (segment (start 134.35 84.35) (end 134.35 85.199999) (width 0.3) (layer "F.Cu") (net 2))
 (segment (start 134.35 85.199999) (end 135.375001 86.225) (width 0.3) (layer "F.Cu") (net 2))
 (segment (start 138.75 101) (end 138.75 98.25) (width 2) (layer "F.Cu") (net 2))
 (segment (start 148.46 86.46) (end 148.46 88.5) (width 0.3) (layer "F.Cu") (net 2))
 (segment (start 135.375001 86.225) (end 138.775 86.225) (width 0.3) (layer "F.Cu") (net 2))
 (segment (start 138.75 98.25) (end 141.5 95.5) (width 2) (layer "F.Cu") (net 2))
 (segment (start 147.65 85.65) (end 148.46 86.46) (width 0.3) (layer "F.Cu") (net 2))
 (segment (start 139.35 85.65) (end 147.65 85.65) (width 0.3) (layer "F.Cu") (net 2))
 (segment (start 163.25 101) (end 163.25 98.25) (width 2) (layer "F.Cu") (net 3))
 (segment (start 135.6 85.199999) (end 136.125001 85.725) (width 0.3) (layer "F.Cu") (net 3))
 (segment (start 163.25 98.25) (end 160.5 95.5) (width 2) (layer "F.Cu") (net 3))
 (segment (start 136.125001 85.725) (end 138.5 85.725) (width 0.3) (layer "F.Cu") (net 3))
 (segment (start 139.3 84.925) (end 152.75 84.925) (width 0.3) (layer "F.Cu") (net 3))
 (segment (start 135.6 84.35) (end 135.6 85.199999) (width 0.3) (layer "F.Cu") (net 3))
 (segment (start 153.54 85.715) (end 153.54 88.5) (width 0.3) (layer "F.Cu") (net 3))
 (segment (start 138.5 85.725) (end 139.3 84.925) (width 0.3) (layer "F.Cu") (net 3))
 (segment (start 152.75 84.925) (end 153.54 85.715) (width 0.3) (layer "F.Cu") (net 3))
 (segment (start 148.75 101) (end 146.5 98.75) (width 2) (layer "B.Cu") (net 1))
 (segment (start 153.25 101) (end 155.5 98.75) (width 2) (layer "B.Cu") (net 1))
 (segment (start 146.5 98.75) (end 131.5 98.75) (width 2) (layer "B.Cu") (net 1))
 (segment (start 155.5 98.75) (end 169.75 98.75) (width 2) (layer "B.Cu") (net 1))
 (segment (start 153.25 101) (end 148.75 101) (width 2) (layer "B.Cu") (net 1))
 (segment (start 129.5 100.75) (end 119.5 100.75) (width 2) (layer "B.Cu") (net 1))
 (segment (start 131.5 98.75) (end 129.5 100.75) (width 2) (layer "B.Cu") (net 1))
 (segment (start 169.75 98.75) (end 171.75 100.75) (width 2) (layer "B.Cu") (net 1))
 (segment (start 171.75 100.75) (end 182.5 100.75) (width 2) (layer "B.Cu") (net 1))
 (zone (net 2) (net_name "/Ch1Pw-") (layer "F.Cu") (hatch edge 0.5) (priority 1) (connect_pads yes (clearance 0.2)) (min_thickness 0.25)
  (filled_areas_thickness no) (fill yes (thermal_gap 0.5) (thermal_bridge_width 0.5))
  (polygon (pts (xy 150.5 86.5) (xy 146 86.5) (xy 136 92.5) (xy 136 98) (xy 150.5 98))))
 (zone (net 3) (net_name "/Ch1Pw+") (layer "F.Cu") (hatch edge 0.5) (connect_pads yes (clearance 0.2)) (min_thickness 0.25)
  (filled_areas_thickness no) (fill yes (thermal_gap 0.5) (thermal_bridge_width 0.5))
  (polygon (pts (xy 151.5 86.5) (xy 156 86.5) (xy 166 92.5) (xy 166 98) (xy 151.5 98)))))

